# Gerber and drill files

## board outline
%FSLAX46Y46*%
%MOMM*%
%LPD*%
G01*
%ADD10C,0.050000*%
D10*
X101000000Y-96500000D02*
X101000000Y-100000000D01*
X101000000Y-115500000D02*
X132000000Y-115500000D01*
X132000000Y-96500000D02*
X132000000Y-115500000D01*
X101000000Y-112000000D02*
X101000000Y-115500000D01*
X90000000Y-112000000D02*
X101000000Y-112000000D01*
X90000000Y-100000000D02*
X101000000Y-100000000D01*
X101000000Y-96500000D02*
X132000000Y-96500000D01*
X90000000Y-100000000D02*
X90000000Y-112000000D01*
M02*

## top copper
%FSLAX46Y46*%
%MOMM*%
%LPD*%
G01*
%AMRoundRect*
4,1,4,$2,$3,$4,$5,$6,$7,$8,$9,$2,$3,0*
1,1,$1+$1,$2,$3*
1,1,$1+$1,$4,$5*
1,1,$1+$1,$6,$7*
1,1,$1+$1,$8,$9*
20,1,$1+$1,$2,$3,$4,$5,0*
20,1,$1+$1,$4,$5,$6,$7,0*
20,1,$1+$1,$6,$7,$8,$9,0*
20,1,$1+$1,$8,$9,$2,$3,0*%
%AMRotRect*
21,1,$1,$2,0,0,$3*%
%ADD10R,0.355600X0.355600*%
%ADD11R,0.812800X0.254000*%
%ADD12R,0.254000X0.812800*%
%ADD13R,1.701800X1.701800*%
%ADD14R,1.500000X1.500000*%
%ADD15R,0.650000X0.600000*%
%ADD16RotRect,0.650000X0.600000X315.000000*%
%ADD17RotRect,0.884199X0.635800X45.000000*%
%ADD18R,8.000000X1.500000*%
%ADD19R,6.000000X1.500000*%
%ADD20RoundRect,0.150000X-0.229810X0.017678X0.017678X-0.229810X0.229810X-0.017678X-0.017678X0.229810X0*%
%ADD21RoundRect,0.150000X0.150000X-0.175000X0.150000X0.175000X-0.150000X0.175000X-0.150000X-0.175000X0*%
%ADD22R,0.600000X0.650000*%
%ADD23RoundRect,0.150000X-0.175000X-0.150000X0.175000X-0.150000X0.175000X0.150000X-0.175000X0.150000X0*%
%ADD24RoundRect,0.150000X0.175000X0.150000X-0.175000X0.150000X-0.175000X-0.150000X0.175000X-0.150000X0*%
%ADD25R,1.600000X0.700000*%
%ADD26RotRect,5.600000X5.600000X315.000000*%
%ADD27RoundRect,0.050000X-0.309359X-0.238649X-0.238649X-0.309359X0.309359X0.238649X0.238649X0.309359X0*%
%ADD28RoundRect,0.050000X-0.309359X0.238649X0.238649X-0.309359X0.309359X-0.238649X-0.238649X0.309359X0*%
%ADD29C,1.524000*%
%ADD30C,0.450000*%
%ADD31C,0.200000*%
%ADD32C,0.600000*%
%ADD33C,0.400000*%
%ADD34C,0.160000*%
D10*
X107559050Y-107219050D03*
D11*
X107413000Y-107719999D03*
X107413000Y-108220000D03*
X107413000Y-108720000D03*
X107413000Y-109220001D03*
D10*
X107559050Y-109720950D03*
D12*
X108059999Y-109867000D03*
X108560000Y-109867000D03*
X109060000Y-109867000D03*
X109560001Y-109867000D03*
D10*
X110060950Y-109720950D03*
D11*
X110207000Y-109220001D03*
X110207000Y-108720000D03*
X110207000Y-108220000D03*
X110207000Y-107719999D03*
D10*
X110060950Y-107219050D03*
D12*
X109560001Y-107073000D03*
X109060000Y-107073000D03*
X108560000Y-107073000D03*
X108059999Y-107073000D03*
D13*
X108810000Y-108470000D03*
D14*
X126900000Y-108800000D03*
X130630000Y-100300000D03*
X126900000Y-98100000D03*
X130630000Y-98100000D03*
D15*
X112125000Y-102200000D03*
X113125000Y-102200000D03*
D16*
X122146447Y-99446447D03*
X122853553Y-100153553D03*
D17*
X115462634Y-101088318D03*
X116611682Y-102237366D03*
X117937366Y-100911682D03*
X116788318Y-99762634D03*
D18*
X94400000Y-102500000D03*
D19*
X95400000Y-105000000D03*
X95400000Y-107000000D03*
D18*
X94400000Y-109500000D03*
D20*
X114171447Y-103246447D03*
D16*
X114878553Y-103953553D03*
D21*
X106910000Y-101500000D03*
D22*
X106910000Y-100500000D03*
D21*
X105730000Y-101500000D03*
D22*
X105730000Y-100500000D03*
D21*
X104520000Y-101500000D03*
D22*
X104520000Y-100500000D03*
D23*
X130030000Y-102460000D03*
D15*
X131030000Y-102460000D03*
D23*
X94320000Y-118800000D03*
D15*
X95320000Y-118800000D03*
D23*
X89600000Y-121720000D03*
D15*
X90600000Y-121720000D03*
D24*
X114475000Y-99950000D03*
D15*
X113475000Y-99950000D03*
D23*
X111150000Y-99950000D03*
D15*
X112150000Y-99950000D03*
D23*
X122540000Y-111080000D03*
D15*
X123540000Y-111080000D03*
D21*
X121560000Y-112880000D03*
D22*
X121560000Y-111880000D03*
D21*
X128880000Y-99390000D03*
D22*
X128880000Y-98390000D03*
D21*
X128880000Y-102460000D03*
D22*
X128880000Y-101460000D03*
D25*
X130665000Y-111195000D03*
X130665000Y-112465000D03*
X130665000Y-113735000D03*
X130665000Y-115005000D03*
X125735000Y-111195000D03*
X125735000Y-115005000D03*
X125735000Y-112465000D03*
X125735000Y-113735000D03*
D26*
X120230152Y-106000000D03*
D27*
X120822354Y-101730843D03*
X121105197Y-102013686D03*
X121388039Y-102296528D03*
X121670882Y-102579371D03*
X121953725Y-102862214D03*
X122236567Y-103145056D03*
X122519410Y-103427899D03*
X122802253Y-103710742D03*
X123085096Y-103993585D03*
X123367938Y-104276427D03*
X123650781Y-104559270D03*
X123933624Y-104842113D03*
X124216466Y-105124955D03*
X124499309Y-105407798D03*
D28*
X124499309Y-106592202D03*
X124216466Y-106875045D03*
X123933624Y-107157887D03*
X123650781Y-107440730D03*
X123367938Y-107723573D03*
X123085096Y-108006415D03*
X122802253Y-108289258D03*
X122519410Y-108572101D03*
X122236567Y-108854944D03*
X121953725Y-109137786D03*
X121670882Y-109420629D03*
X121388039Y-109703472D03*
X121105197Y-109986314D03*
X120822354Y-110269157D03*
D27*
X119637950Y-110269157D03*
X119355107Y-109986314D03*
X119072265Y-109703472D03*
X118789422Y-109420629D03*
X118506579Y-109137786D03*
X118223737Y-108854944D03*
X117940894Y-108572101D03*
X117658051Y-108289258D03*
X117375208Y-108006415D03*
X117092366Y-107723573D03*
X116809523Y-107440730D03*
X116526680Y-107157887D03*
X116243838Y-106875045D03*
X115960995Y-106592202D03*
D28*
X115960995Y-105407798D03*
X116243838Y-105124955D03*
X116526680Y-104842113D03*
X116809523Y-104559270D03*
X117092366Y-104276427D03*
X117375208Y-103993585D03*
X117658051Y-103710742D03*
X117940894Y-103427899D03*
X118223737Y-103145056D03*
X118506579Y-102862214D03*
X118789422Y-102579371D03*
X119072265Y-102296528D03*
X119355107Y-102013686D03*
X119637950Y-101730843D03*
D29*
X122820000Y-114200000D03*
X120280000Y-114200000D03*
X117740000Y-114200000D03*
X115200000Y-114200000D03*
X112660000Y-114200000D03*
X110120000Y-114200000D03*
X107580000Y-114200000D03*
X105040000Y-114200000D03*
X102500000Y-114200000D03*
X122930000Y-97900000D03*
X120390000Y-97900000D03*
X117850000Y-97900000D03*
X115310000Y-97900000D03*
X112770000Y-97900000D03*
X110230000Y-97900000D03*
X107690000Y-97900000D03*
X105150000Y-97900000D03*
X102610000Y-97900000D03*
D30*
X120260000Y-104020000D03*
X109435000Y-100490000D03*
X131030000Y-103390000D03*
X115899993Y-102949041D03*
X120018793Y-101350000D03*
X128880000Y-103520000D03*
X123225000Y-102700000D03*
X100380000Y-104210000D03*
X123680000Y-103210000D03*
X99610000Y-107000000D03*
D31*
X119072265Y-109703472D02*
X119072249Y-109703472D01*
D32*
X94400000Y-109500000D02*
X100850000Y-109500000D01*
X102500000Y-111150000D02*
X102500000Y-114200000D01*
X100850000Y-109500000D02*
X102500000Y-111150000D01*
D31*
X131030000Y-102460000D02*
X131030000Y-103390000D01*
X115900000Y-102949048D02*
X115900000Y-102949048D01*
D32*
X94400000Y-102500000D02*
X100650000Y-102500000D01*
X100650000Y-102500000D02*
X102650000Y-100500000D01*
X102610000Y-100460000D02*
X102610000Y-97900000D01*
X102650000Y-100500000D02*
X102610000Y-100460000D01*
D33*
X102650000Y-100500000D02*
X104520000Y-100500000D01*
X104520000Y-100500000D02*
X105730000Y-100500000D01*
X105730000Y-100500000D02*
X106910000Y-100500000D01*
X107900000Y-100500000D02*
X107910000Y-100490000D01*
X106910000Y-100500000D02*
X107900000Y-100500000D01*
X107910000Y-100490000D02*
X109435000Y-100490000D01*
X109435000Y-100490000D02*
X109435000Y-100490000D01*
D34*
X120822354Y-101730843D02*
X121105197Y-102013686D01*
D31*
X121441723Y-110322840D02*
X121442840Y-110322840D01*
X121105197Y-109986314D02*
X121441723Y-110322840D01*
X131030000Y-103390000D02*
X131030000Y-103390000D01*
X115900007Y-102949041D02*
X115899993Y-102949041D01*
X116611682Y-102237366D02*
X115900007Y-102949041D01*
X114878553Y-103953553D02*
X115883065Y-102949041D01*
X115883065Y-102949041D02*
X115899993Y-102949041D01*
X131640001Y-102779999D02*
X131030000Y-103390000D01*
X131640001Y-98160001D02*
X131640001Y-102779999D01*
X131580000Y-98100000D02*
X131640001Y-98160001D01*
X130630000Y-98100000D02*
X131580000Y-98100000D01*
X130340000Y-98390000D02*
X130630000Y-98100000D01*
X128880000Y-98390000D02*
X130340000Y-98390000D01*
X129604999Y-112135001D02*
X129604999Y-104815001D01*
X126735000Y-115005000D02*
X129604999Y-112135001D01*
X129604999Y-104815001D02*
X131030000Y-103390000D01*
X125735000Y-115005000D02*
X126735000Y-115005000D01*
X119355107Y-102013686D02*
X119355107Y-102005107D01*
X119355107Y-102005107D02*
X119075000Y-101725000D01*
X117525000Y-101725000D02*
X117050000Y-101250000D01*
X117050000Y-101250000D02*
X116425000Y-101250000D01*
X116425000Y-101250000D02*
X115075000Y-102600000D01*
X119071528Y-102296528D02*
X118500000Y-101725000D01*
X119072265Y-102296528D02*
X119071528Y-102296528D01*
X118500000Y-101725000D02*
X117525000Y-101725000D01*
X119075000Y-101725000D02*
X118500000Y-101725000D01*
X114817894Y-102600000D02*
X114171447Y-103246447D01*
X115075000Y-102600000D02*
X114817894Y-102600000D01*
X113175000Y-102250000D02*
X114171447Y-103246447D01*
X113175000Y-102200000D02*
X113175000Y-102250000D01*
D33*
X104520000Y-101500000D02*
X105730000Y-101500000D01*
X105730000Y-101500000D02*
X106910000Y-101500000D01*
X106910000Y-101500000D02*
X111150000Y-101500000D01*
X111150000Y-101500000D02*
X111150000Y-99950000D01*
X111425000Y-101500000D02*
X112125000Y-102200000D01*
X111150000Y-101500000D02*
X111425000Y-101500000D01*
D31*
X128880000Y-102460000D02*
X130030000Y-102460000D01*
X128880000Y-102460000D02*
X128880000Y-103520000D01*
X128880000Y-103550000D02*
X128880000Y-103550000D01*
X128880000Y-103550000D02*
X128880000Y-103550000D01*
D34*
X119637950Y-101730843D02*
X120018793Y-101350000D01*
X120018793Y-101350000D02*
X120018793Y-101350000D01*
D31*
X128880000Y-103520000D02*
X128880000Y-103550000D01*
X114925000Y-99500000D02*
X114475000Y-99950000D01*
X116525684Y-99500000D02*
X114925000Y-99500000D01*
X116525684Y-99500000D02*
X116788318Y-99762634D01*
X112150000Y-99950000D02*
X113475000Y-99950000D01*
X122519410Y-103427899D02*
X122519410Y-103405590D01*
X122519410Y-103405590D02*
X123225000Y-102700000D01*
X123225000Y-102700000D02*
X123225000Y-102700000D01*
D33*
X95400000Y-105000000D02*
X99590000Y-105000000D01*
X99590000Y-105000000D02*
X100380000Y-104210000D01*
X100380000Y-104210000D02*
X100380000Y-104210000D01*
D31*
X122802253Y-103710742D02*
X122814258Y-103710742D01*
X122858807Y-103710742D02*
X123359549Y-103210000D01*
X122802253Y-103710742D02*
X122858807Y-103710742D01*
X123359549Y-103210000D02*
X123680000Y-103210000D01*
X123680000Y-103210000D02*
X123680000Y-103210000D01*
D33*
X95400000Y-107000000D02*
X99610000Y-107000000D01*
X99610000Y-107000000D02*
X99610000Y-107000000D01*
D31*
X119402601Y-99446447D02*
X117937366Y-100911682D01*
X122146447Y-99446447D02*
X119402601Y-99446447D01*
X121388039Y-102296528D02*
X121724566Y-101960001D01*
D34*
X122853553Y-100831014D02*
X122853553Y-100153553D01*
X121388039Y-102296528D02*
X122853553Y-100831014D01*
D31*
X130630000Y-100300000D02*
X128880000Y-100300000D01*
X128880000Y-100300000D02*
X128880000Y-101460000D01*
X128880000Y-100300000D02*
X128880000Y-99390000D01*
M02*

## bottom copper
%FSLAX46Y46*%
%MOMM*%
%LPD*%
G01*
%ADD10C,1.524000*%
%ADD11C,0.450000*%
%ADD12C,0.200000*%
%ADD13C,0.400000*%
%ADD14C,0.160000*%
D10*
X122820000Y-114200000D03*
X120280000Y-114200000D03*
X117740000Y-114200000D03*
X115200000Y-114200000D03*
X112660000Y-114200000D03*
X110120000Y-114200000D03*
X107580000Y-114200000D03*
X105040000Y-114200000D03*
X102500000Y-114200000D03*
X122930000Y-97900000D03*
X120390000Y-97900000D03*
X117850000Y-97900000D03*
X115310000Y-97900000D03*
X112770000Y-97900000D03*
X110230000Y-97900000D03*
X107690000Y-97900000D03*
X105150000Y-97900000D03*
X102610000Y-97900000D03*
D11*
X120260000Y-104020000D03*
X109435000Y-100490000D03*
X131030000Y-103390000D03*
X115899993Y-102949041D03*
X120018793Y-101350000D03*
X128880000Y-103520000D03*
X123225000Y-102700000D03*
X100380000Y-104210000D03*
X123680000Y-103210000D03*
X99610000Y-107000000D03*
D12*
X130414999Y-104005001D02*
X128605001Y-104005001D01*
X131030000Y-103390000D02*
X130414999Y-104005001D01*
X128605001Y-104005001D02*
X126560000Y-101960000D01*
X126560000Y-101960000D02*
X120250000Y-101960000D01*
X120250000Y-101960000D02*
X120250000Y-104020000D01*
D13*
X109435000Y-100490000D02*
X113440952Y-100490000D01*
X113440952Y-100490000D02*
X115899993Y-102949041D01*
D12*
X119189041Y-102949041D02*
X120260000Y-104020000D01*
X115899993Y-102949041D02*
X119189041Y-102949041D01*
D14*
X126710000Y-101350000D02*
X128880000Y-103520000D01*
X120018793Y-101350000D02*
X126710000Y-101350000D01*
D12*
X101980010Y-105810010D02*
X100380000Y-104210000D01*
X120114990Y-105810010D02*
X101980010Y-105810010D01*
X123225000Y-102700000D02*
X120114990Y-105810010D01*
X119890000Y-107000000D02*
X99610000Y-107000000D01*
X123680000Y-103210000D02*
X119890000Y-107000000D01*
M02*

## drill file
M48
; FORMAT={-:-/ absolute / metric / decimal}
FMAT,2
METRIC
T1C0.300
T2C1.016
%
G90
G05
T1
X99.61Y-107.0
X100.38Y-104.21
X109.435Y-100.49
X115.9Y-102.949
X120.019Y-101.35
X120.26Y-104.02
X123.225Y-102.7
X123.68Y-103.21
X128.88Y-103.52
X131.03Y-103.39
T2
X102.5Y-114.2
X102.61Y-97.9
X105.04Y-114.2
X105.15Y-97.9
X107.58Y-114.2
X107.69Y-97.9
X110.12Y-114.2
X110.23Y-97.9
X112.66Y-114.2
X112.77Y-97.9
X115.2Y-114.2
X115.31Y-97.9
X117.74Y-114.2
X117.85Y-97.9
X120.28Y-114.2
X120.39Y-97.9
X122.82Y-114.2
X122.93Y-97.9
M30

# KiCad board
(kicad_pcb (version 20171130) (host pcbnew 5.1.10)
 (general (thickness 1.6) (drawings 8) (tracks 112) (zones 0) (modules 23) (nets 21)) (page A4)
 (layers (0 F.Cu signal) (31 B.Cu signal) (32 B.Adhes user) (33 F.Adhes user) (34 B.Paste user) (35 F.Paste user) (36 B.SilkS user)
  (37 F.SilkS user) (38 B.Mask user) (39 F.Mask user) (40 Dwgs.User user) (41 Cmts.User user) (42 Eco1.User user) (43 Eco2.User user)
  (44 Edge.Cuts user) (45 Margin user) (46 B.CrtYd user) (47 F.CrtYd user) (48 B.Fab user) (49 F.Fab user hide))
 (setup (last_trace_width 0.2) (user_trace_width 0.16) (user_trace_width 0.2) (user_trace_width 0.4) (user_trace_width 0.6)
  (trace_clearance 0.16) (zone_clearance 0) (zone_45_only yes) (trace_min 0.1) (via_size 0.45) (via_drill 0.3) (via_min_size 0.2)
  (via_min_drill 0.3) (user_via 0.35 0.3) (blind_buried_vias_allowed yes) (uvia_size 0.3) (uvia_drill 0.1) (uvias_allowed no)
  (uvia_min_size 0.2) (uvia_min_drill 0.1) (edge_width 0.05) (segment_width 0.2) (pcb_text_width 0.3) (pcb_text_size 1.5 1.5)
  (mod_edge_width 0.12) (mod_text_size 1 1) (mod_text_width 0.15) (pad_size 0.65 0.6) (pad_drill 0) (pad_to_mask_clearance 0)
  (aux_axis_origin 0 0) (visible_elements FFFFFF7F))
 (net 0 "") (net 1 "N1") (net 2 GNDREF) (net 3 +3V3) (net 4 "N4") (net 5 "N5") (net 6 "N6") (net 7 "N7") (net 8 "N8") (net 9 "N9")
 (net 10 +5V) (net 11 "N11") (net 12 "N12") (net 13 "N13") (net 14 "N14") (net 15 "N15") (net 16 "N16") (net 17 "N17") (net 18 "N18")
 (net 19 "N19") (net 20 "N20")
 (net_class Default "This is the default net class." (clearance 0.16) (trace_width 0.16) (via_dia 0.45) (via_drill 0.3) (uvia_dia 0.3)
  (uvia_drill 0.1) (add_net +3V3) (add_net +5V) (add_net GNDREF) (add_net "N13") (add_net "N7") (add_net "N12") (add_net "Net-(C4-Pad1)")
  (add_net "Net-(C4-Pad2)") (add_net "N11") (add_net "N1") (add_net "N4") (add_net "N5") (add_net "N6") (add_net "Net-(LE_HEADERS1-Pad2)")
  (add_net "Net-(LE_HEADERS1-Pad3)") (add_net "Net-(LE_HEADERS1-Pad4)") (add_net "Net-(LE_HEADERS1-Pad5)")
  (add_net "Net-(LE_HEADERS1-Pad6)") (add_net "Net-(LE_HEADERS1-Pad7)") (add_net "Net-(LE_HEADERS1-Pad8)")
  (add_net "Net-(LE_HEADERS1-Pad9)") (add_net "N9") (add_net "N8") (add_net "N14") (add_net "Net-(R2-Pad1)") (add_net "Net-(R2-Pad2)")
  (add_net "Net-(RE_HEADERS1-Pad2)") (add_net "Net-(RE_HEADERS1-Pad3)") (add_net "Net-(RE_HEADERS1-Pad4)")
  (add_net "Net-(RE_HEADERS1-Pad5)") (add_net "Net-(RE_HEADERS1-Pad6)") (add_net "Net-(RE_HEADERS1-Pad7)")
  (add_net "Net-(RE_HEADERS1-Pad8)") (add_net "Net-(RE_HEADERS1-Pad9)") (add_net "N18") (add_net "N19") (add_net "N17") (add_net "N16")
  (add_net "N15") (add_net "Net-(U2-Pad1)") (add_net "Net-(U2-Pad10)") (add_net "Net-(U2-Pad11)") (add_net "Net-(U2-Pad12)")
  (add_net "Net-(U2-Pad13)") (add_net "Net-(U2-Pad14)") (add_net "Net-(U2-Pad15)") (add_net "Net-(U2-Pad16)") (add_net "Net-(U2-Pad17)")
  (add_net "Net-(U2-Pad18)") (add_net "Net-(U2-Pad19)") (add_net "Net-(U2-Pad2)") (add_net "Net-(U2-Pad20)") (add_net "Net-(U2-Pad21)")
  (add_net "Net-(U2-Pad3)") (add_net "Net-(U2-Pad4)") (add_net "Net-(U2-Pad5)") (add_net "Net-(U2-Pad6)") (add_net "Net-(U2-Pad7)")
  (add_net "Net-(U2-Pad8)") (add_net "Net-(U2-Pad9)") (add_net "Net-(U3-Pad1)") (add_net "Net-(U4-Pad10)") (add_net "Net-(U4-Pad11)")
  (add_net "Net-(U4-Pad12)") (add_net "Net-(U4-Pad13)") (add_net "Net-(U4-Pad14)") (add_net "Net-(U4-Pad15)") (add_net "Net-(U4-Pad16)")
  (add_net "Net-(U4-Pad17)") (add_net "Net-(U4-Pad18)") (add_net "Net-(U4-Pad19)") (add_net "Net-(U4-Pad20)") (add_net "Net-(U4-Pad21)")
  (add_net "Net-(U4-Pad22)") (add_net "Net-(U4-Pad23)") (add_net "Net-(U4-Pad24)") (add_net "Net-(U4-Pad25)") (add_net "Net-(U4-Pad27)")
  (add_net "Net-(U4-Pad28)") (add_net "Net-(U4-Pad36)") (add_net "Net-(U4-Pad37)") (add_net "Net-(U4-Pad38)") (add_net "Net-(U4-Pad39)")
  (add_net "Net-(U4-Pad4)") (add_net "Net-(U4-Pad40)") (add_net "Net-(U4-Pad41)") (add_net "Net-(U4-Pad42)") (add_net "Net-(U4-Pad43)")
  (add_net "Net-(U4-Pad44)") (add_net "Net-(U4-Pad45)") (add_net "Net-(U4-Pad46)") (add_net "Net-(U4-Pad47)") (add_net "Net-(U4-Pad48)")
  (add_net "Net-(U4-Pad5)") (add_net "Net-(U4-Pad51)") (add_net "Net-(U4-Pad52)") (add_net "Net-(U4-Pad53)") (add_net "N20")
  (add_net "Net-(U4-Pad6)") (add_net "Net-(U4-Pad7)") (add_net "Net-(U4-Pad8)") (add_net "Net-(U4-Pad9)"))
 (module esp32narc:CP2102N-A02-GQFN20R (layer F.Cu) (at 108.81 108.47)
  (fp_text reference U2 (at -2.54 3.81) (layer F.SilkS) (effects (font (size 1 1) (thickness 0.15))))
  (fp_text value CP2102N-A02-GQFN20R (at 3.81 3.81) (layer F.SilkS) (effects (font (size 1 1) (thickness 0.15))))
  (pad 1 smd rect (at -1.25095 -1.25095) (size 0.3556 0.3556) (layers F.Cu F.Paste F.Mask))
  (pad 2 smd rect (at -1.397 -0.750001 90) (size 0.254 0.8128) (layers F.Cu F.Paste F.Mask))
  (pad 3 smd rect (at -1.397 -0.25 90) (size 0.254 0.8128) (layers F.Cu F.Paste F.Mask))
  (pad 4 smd rect (at -1.397 0.25 90) (size 0.254 0.8128) (layers F.Cu F.Paste F.Mask))
  (pad 5 smd rect (at -1.397 0.750001 90) (size 0.254 0.8128) (layers F.Cu F.Paste F.Mask))
  (pad 6 smd rect (at -1.25095 1.25095) (size 0.3556 0.3556) (layers F.Cu F.Paste F.Mask))
  (pad 7 smd rect (at -0.750001 1.397) (size 0.254 0.8128) (layers F.Cu F.Paste F.Mask))
  (pad 8 smd rect (at -0.25 1.397) (size 0.254 0.8128) (layers F.Cu F.Paste F.Mask))
  (pad 9 smd rect (at 0.25 1.397) (size 0.254 0.8128) (layers F.Cu F.Paste F.Mask))
  (pad 10 smd rect (at 0.750001 1.397) (size 0.254 0.8128) (layers F.Cu F.Paste F.Mask))
  (pad 11 smd rect (at 1.25095 1.25095) (size 0.3556 0.3556) (layers F.Cu F.Paste F.Mask))
  (pad 12 smd rect (at 1.397 0.750001 90) (size 0.254 0.8128) (layers F.Cu F.Paste F.Mask))
  (pad 13 smd rect (at 1.397 0.25 90) (size 0.254 0.8128) (layers F.Cu F.Paste F.Mask))
  (pad 14 smd rect (at 1.397 -0.25 90) (size 0.254 0.8128) (layers F.Cu F.Paste F.Mask))
  (pad 15 smd rect (at 1.397 -0.750001 90) (size 0.254 0.8128) (layers F.Cu F.Paste F.Mask))
  (pad 16 smd rect (at 1.25095 -1.25095) (size 0.3556 0.3556) (layers F.Cu F.Paste F.Mask))
  (pad 17 smd rect (at 0.750001 -1.397) (size 0.254 0.8128) (layers F.Cu F.Paste F.Mask))
  (pad 18 smd rect (at 0.25 -1.397) (size 0.254 0.8128) (layers F.Cu F.Paste F.Mask))
  (pad 19 smd rect (at -0.25 -1.397) (size 0.254 0.8128) (layers F.Cu F.Paste F.Mask))
  (pad 20 smd rect (at -0.750001 -1.397) (size 0.254 0.8128) (layers F.Cu F.Paste F.Mask))
  (pad 21 smd rect (at 0 0) (size 1.7018 1.7018) (layers F.Cu F.Paste F.Mask)))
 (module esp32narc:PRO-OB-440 (layer F.Cu) (at 130.63 98.1 270)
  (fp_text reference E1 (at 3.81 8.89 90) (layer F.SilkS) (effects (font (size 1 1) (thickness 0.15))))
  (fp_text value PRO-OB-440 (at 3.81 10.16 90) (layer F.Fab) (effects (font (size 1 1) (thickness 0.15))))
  (pad 4 smd rect (at 10.7 3.73 270) (size 1.5 1.5) (layers F.Cu F.Paste F.Mask) (clearance 0.75))
  (pad 2 smd rect (at 2.2 0 270) (size 1.5 1.5) (layers F.Cu F.Paste F.Mask) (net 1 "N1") (clearance 0.15))
  (pad 3 smd rect (at 0 3.73 270) (size 1.5 1.5) (layers F.Cu F.Paste F.Mask) (clearance 0.55))
  (pad 1 smd rect (at 0 0 270) (size 1.5 1.5) (layers F.Cu F.Paste F.Mask) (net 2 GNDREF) (clearance 0.15)))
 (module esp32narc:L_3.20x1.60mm (layer F.Cu) (at 112.625 102.2)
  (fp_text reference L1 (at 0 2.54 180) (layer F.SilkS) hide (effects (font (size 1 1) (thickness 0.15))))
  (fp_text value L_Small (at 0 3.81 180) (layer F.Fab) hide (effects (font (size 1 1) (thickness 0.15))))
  (pad 1 smd rect (at -0.5 0) (size 0.65 0.6) (layers F.Cu F.Paste F.Mask) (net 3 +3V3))
  (pad 2 smd rect (at 0.5 0) (size 0.65 0.6) (layers F.Cu F.Paste F.Mask) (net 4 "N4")))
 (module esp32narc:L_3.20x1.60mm (layer F.Cu) (at 122.5 99.8 315)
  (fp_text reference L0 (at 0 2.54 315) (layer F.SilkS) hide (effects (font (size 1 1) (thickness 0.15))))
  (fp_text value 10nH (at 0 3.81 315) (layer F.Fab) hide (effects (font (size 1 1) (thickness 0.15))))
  (pad 1 smd rect (at -0.5 0 315) (size 0.65 0.6) (layers F.Cu F.Paste F.Mask) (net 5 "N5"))
  (pad 2 smd rect (at 0.5 0 315) (size 0.65 0.6) (layers F.Cu F.Paste F.Mask) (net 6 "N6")))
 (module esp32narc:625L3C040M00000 (layer F.Cu) (at 116.7 101 45)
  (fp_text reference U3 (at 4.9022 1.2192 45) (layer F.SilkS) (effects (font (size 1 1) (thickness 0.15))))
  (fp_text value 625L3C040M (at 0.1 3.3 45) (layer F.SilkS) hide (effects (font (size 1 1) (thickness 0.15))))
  (pad 1 smd rect (at -0.9374 -0.8125 45) (size 0.884199 0.6358) (layers F.Cu F.Paste F.Mask))
  (pad 2 smd rect (at -0.9374 0.8125 45) (size 0.884199 0.6358) (layers F.Cu F.Paste F.Mask) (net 2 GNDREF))
  (pad 3 smd rect (at 0.9374 0.8125 45) (size 0.884199 0.6358) (layers F.Cu F.Paste F.Mask) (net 5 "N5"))
  (pad 4 smd rect (at 0.9374 -0.8125 45) (size 0.884199 0.6358) (layers F.Cu F.Paste F.Mask) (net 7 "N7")))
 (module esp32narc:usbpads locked (layer F.Cu) (at 98.4 106 90)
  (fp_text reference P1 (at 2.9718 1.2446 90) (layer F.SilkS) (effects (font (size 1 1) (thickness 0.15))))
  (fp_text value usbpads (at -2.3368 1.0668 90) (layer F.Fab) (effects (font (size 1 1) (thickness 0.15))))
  (pad P4 smd rect (at 3.5 -4 90) (size 1.5 8) (layers F.Cu F.Paste F.Mask) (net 2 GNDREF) (solder_mask_margin 0.105) (clearance 0.55))
  (pad P3 smd rect (at 1 -3 90) (size 1.5 6) (layers F.Cu F.Paste F.Mask) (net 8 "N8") (clearance 0.55))
  (pad P2 smd rect (at -1 -3 90) (size 1.5 6) (layers F.Cu F.Paste F.Mask) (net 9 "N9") (clearance 0.55))
  (pad P1 smd rect (at -3.5 -4 90) (size 1.5 8) (layers F.Cu F.Paste F.Mask) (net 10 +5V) (solder_mask_margin 0.105) (clearance 0.55)))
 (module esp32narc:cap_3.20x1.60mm (layer F.Cu) (at 114.525 103.6 315)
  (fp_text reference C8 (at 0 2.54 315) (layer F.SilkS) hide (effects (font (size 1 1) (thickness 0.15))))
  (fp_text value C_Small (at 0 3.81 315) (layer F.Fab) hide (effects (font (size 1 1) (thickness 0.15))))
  (pad 1 smd roundrect (at -0.5 0 315) (size 0.65 0.6) (layers F.Cu F.Paste F.Mask) (roundrect_rratio 0.25) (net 4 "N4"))
  (pad 2 smd rect (at 0.5 0 315) (size 0.65 0.6) (layers F.Cu F.Paste F.Mask) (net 2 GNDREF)))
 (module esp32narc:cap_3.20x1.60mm (layer F.Cu) (at 106.91 101 90)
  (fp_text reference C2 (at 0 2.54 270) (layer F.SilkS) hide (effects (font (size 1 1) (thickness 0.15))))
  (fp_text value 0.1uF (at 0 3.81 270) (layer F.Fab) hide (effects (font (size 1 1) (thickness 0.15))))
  (pad 1 smd roundrect (at -0.5 0 90) (size 0.65 0.6) (layers F.Cu F.Paste F.Mask) (roundrect_rratio 0.25) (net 3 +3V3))
  (pad 2 smd rect (at 0.5 0 90) (size 0.65 0.6) (layers F.Cu F.Paste F.Mask) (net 2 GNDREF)))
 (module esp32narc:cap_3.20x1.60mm (layer F.Cu) (at 105.73 101 90)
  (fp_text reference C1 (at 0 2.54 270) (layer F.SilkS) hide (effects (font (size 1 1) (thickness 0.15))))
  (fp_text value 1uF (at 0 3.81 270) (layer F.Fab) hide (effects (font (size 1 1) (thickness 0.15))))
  (pad 1 smd roundrect (at -0.5 0 90) (size 0.65 0.6) (layers F.Cu F.Paste F.Mask) (roundrect_rratio 0.25) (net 3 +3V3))
  (pad 2 smd rect (at 0.5 0 90) (size 0.65 0.6) (layers F.Cu F.Paste F.Mask) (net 2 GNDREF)))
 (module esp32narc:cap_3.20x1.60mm (layer F.Cu) (at 104.52 101 90)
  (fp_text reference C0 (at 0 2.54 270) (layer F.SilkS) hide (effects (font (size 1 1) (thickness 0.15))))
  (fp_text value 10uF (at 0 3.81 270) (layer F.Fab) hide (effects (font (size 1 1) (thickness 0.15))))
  (pad 1 smd roundrect (at -0.5 0 90) (size 0.65 0.6) (layers F.Cu F.Paste F.Mask) (roundrect_rratio 0.25) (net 3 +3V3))
  (pad 2 smd rect (at 0.5 0 90) (size 0.65 0.6) (layers F.Cu F.Paste F.Mask) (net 2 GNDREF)))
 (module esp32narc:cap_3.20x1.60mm (layer F.Cu) (at 130.53 102.46)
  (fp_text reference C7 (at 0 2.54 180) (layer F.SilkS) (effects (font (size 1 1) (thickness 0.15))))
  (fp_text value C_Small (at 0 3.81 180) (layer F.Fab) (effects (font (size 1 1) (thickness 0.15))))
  (pad 1 smd roundrect (at -0.5 0) (size 0.65 0.6) (layers F.Cu F.Paste F.Mask) (roundrect_rratio 0.25) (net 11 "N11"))
  (pad 2 smd rect (at 0.5 0) (size 0.65 0.6) (layers F.Cu F.Paste F.Mask) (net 2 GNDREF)))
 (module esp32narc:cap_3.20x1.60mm (layer F.Cu) (at 94.82 118.8)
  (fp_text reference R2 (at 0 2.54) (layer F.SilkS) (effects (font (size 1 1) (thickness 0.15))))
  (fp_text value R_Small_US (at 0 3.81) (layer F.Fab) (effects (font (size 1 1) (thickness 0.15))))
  (pad 1 smd roundrect (at -0.5 0) (size 0.65 0.6) (layers F.Cu F.Paste F.Mask) (roundrect_rratio 0.25))
  (pad 2 smd rect (at 0.5 0) (size 0.65 0.6) (layers F.Cu F.Paste F.Mask)))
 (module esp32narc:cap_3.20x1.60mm (layer F.Cu) (at 90.1 121.72)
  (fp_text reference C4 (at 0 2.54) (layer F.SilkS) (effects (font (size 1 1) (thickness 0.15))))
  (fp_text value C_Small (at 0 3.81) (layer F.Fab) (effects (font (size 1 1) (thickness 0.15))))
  (pad 1 smd roundrect (at -0.5 0) (size 0.65 0.6) (layers F.Cu F.Paste F.Mask) (roundrect_rratio 0.25))
  (pad 2 smd rect (at 0.5 0) (size 0.65 0.6) (layers F.Cu F.Paste F.Mask)))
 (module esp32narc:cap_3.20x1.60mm (layer F.Cu) (at 113.975 99.95 180)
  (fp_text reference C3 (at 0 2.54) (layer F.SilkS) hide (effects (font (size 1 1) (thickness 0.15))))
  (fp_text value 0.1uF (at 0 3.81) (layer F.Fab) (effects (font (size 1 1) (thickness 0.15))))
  (pad 1 smd roundrect (at -0.5 0 180) (size 0.65 0.6) (layers F.Cu F.Paste F.Mask) (roundrect_rratio 0.25) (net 7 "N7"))
  (pad 2 smd rect (at 0.5 0 180) (size 0.65 0.6) (layers F.Cu F.Paste F.Mask) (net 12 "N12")))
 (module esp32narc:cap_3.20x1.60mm (layer F.Cu) (at 111.65 99.95)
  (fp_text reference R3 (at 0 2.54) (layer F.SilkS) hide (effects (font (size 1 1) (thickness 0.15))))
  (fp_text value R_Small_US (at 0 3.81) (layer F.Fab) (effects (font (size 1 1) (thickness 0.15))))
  (pad 1 smd roundrect (at -0.5 0) (size 0.65 0.6) (layers F.Cu F.Paste F.Mask) (roundrect_rratio 0.25) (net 3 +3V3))
  (pad 2 smd rect (at 0.5 0) (size 0.65 0.6) (layers F.Cu F.Paste F.Mask) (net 12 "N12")))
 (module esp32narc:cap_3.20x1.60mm (layer F.Cu) (at 123.04 111.08)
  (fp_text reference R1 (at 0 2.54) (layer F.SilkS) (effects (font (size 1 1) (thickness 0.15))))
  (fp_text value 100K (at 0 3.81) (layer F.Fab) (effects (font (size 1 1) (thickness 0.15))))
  (pad 1 smd roundrect (at -0.5 0) (size 0.65 0.6) (layers F.Cu F.Paste F.Mask) (roundrect_rratio 0.25) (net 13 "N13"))
  (pad 2 smd rect (at 0.5 0) (size 0.65 0.6) (layers F.Cu F.Paste F.Mask) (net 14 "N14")))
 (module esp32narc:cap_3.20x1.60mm (layer F.Cu) (at 121.56 112.38 90)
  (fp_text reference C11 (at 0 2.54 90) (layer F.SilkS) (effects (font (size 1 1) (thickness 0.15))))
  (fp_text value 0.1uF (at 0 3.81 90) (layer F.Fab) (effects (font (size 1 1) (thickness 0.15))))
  (pad 1 smd roundrect (at -0.5 0 90) (size 0.65 0.6) (layers F.Cu F.Paste F.Mask) (roundrect_rratio 0.25) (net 2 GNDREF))
  (pad 2 smd rect (at 0.5 0 90) (size 0.65 0.6) (layers F.Cu F.Paste F.Mask) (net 13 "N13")))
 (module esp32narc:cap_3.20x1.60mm (layer F.Cu) (at 128.88 98.89 90)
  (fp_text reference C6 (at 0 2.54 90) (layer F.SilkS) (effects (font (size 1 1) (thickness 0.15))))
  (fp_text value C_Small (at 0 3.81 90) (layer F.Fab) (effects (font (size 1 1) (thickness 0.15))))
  (pad 1 smd roundrect (at -0.5 0 90) (size 0.65 0.6) (layers F.Cu F.Paste F.Mask) (roundrect_rratio 0.25) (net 1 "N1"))
  (pad 2 smd rect (at 0.5 0 90) (size 0.65 0.6) (layers F.Cu F.Paste F.Mask) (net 2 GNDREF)))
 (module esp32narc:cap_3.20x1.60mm (layer F.Cu) (at 128.88 101.96 90)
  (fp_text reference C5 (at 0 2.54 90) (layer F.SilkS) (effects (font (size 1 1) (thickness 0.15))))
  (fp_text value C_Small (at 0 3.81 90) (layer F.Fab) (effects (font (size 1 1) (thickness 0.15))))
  (pad 1 smd roundrect (at -0.5 0 90) (size 0.65 0.6) (layers F.Cu F.Paste F.Mask) (roundrect_rratio 0.25) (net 11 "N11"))
  (pad 2 smd rect (at 0.5 0 90) (size 0.65 0.6) (layers F.Cu F.Paste F.Mask) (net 1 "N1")))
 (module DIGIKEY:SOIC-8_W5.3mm (layer F.Cu) (at 128.2 113.1)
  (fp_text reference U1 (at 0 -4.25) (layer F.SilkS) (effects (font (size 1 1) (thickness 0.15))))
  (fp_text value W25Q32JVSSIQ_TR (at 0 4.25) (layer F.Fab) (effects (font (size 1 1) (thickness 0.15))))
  (pad 8 smd rect (at 2.465 -1.905) (size 1.6 0.7) (layers F.Cu F.Paste F.Mask) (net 13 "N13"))
  (pad 7 smd rect (at 2.465 -0.635) (size 1.6 0.7) (layers F.Cu F.Paste F.Mask) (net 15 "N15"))
  (pad 6 smd rect (at 2.465 0.635) (size 1.6 0.7) (layers F.Cu F.Paste F.Mask) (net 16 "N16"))
  (pad 5 smd rect (at 2.465 1.905) (size 1.6 0.7) (layers F.Cu F.Paste F.Mask) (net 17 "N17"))
  (pad 1 smd rect (at -2.465 -1.905) (size 1.6 0.7) (layers F.Cu F.Paste F.Mask) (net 14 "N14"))
  (pad 4 smd rect (at -2.465 1.905) (size 1.6 0.7) (layers F.Cu F.Paste F.Mask) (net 2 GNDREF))
  (pad 2 smd rect (at -2.465 -0.635) (size 1.6 0.7) (layers F.Cu F.Paste F.Mask) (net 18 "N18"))
  (pad 3 smd rect (at -2.465 0.635) (size 1.6 0.7) (layers F.Cu F.Paste F.Mask) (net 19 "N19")))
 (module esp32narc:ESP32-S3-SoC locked (layer F.Cu) (at 120.230152 106 315)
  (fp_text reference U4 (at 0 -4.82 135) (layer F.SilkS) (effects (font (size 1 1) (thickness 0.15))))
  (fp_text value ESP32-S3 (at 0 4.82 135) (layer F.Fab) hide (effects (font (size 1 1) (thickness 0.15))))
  (pad "" smd roundrect (at 2.1 2.1 315) (size 1.13 1.13) (layers F.Paste) (roundrect_rratio 0.221239))
  (pad "" smd roundrect (at 2.1 0.7 315) (size 1.13 1.13) (layers F.Paste) (roundrect_rratio 0.221239))
  (pad "" smd roundrect (at 2.1 -0.7 315) (size 1.13 1.13) (layers F.Paste) (roundrect_rratio 0.221239))
  (pad "" smd roundrect (at 2.1 -2.1 315) (size 1.13 1.13) (layers F.Paste) (roundrect_rratio 0.221239))
  (pad "" smd roundrect (at 0.7 2.1 315) (size 1.13 1.13) (layers F.Paste) (roundrect_rratio 0.221239))
  (pad "" smd roundrect (at 0.7 0.7 315) (size 1.13 1.13) (layers F.Paste) (roundrect_rratio 0.221239))
  (pad "" smd roundrect (at 0.7 -0.7 315) (size 1.13 1.13) (layers F.Paste) (roundrect_rratio 0.221239))
  (pad "" smd roundrect (at 0.7 -2.1 315) (size 1.13 1.13) (layers F.Paste) (roundrect_rratio 0.221239))
  (pad "" smd roundrect (at -0.7 2.1 315) (size 1.13 1.13) (layers F.Paste) (roundrect_rratio 0.221239))
  (pad "" smd roundrect (at -0.7 0.7 315) (size 1.13 1.13) (layers F.Paste) (roundrect_rratio 0.221239))
  (pad "" smd roundrect (at -0.7 -0.7 315) (size 1.13 1.13) (layers F.Paste) (roundrect_rratio 0.221239))
  (pad "" smd roundrect (at -0.7 -2.1 315) (size 1.13 1.13) (layers F.Paste) (roundrect_rratio 0.221239))
  (pad "" smd roundrect (at -2.1 2.1 315) (size 1.13 1.13) (layers F.Paste) (roundrect_rratio 0.221239))
  (pad "" smd roundrect (at -2.1 0.7 315) (size 1.13 1.13) (layers F.Paste) (roundrect_rratio 0.221239))
  (pad "" smd roundrect (at -2.1 -0.7 315) (size 1.13 1.13) (layers F.Paste) (roundrect_rratio 0.221239))
  (pad "" smd roundrect (at -2.1 -2.1 315) (size 1.13 1.13) (layers F.Paste) (roundrect_rratio 0.221239))
  (pad 57 smd rect (at 0 0 315) (size 5.6 5.6) (layers F.Cu F.Mask) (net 2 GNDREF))
  (pad 56 smd roundrect (at -2.6 -3.4375 315) (size 0.2 0.875) (layers F.Cu F.Paste F.Mask) (roundrect_rratio 0.25) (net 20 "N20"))
  (pad 55 smd roundrect (at -2.2 -3.4375 315) (size 0.2 0.875) (layers F.Cu F.Paste F.Mask) (roundrect_rratio 0.25) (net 20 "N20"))
  (pad 54 smd roundrect (at -1.8 -3.4375 315) (size 0.2 0.875) (layers F.Cu F.Paste F.Mask) (roundrect_rratio 0.25) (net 6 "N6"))
  (pad 53 smd roundrect (at -1.4 -3.4375 315) (size 0.2 0.875) (layers F.Cu F.Paste F.Mask) (roundrect_rratio 0.25))
  (pad 52 smd roundrect (at -1 -3.4375 315) (size 0.2 0.875) (layers F.Cu F.Paste F.Mask) (roundrect_rratio 0.25))
  (pad 51 smd roundrect (at -0.6 -3.4375 315) (size 0.2 0.875) (layers F.Cu F.Paste F.Mask) (roundrect_rratio 0.25))
  (pad 50 smd roundrect (at -0.2 -3.4375 315) (size 0.2 0.875) (layers F.Cu F.Paste F.Mask) (roundrect_rratio 0.25) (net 8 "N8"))
  (pad 49 smd roundrect (at 0.2 -3.4375 315) (size 0.2 0.875) (layers F.Cu F.Paste F.Mask) (roundrect_rratio 0.25) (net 9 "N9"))
  (pad 48 smd roundrect (at 0.6 -3.4375 315) (size 0.2 0.875) (layers F.Cu F.Paste F.Mask) (roundrect_rratio 0.25))
  (pad 47 smd roundrect (at 1 -3.4375 315) (size 0.2 0.875) (layers F.Cu F.Paste F.Mask) (roundrect_rratio 0.25))
  (pad 46 smd roundrect (at 1.4 -3.4375 315) (size 0.2 0.875) (layers F.Cu F.Paste F.Mask) (roundrect_rratio 0.25))
  (pad 45 smd roundrect (at 1.8 -3.4375 315) (size 0.2 0.875) (layers F.Cu F.Paste F.Mask) (roundrect_rratio 0.25))
  (pad 44 smd roundrect (at 2.2 -3.4375 315) (size 0.2 0.875) (layers F.Cu F.Paste F.Mask) (roundrect_rratio 0.25))
  (pad 43 smd roundrect (at 2.6 -3.4375 315) (size 0.2 0.875) (layers F.Cu F.Paste F.Mask) (roundrect_rratio 0.25))
  (pad 42 smd roundrect (at 3.4375 -2.6 315) (size 0.875 0.2) (layers F.Cu F.Paste F.Mask) (roundrect_rratio 0.25))
  (pad 41 smd roundrect (at 3.4375 -2.2 315) (size 0.875 0.2) (layers F.Cu F.Paste F.Mask) (roundrect_rratio 0.25))
  (pad 40 smd roundrect (at 3.4375 -1.8 315) (size 0.875 0.2) (layers F.Cu F.Paste F.Mask) (roundrect_rratio 0.25))
  (pad 39 smd roundrect (at 3.4375 -1.4 315) (size 0.875 0.2) (layers F.Cu F.Paste F.Mask) (roundrect_rratio 0.25))
  (pad 38 smd roundrect (at 3.4375 -1 315) (size 0.875 0.2) (layers F.Cu F.Paste F.Mask) (roundrect_rratio 0.25))
  (pad 37 smd roundrect (at 3.4375 -0.6 315) (size 0.875 0.2) (layers F.Cu F.Paste F.Mask) (roundrect_rratio 0.25))
  (pad 36 smd roundrect (at 3.4375 -0.2 315) (size 0.875 0.2) (layers F.Cu F.Paste F.Mask) (roundrect_rratio 0.25))
  (pad 35 smd roundrect (at 3.4375 0.2 315) (size 0.875 0.2) (layers F.Cu F.Paste F.Mask) (roundrect_rratio 0.25) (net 17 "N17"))
  (pad 34 smd roundrect (at 3.4375 0.6 315) (size 0.875 0.2) (layers F.Cu F.Paste F.Mask) (roundrect_rratio 0.25) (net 18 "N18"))
  (pad 33 smd roundrect (at 3.4375 1 315) (size 0.875 0.2) (layers F.Cu F.Paste F.Mask) (roundrect_rratio 0.25) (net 16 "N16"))
  (pad 32 smd roundrect (at 3.4375 1.4 315) (size 0.875 0.2) (layers F.Cu F.Paste F.Mask) (roundrect_rratio 0.25) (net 14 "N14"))
  (pad 31 smd roundrect (at 3.4375 1.8 315) (size 0.875 0.2) (layers F.Cu F.Paste F.Mask) (roundrect_rratio 0.25) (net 19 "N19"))
  (pad 30 smd roundrect (at 3.4375 2.2 315) (size 0.875 0.2) (layers F.Cu F.Paste F.Mask) (roundrect_rratio 0.25) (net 15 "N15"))
  (pad 29 smd roundrect (at 3.4375 2.6 315) (size 0.875 0.2) (layers F.Cu F.Paste F.Mask) (roundrect_rratio 0.25) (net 13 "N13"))
  (pad 28 smd roundrect (at 2.6 3.4375 315) (size 0.2 0.875) (layers F.Cu F.Paste F.Mask) (roundrect_rratio 0.25))
  (pad 27 smd roundrect (at 2.2 3.4375 315) (size 0.2 0.875) (layers F.Cu F.Paste F.Mask) (roundrect_rratio 0.25))
  (pad 26 smd roundrect (at 1.8 3.4375 315) (size 0.2 0.875) (layers F.Cu F.Paste F.Mask) (roundrect_rratio 0.25))
  (pad 25 smd roundrect (at 1.4 3.4375 315) (size 0.2 0.875) (layers F.Cu F.Paste F.Mask) (roundrect_rratio 0.25))
  (pad 24 smd roundrect (at 1 3.4375 315) (size 0.2 0.875) (layers F.Cu F.Paste F.Mask) (roundrect_rratio 0.25))
  (pad 23 smd roundrect (at 0.6 3.4375 315) (size 0.2 0.875) (layers F.Cu F.Paste F.Mask) (roundrect_rratio 0.25))
  (pad 22 smd roundrect (at 0.2 3.4375 315) (size 0.2 0.875) (layers F.Cu F.Paste F.Mask) (roundrect_rratio 0.25))
  (pad 21 smd roundrect (at -0.2 3.4375 315) (size 0.2 0.875) (layers F.Cu F.Paste F.Mask) (roundrect_rratio 0.25))
  (pad 20 smd roundrect (at -0.6 3.4375 315) (size 0.2 0.875) (layers F.Cu F.Paste F.Mask) (roundrect_rratio 0.25))
  (pad 19 smd roundrect (at -1 3.4375 315) (size 0.2 0.875) (layers F.Cu F.Paste F.Mask) (roundrect_rratio 0.25))
  (pad 18 smd roundrect (at -1.4 3.4375 315) (size 0.2 0.875) (layers F.Cu F.Paste F.Mask) (roundrect_rratio 0.25))
  (pad 17 smd roundrect (at -1.8 3.4375 315) (size 0.2 0.875) (layers F.Cu F.Paste F.Mask) (roundrect_rratio 0.25))
  (pad 16 smd roundrect (at -2.2 3.4375 315) (size 0.2 0.875) (layers F.Cu F.Paste F.Mask) (roundrect_rratio 0.25))
  (pad 15 smd roundrect (at -2.6 3.4375 315) (size 0.2 0.875) (layers F.Cu F.Paste F.Mask) (roundrect_rratio 0.25))
  (pad 14 smd roundrect (at -3.4375 2.6 315) (size 0.875 0.2) (layers F.Cu F.Paste F.Mask) (roundrect_rratio 0.25))
  (pad 13 smd roundrect (at -3.4375 2.2 315) (size 0.875 0.2) (layers F.Cu F.Paste F.Mask) (roundrect_rratio 0.25))
  (pad 12 smd roundrect (at -3.4375 1.8 315) (size 0.875 0.2) (layers F.Cu F.Paste F.Mask) (roundrect_rratio 0.25))
  (pad 11 smd roundrect (at -3.4375 1.4 315) (size 0.875 0.2) (layers F.Cu F.Paste F.Mask) (roundrect_rratio 0.25))
  (pad 10 smd roundrect (at -3.4375 1 315) (size 0.875 0.2) (layers F.Cu F.Paste F.Mask) (roundrect_rratio 0.25))
  (pad 9 smd roundrect (at -3.4375 0.6 315) (size 0.875 0.2) (layers F.Cu F.Paste F.Mask) (roundrect_rratio 0.25))
  (pad 8 smd roundrect (at -3.4375 0.2 315) (size 0.875 0.2) (layers F.Cu F.Paste F.Mask) (roundrect_rratio 0.25))
  (pad 7 smd roundrect (at -3.4375 -0.2 315) (size 0.875 0.2) (layers F.Cu F.Paste F.Mask) (roundrect_rratio 0.25))
  (pad 6 smd roundrect (at -3.4375 -0.6 315) (size 0.875 0.2) (layers F.Cu F.Paste F.Mask) (roundrect_rratio 0.25))
  (pad 5 smd roundrect (at -3.4375 -1 315) (size 0.875 0.2) (layers F.Cu F.Paste F.Mask) (roundrect_rratio 0.25))
  (pad 4 smd roundrect (at -3.4375 -1.4 315) (size 0.875 0.2) (layers F.Cu F.Paste F.Mask) (roundrect_rratio 0.25))
  (pad 3 smd roundrect (at -3.4375 -1.8 315) (size 0.875 0.2) (layers F.Cu F.Paste F.Mask) (roundrect_rratio 0.25) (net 4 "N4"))
  (pad 2 smd roundrect (at -3.4375 -2.2 315) (size 0.875 0.2) (layers F.Cu F.Paste F.Mask) (roundrect_rratio 0.25) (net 4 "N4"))
  (pad 1 smd roundrect (at -3.4375 -2.6 315) (size 0.875 0.2) (layers F.Cu F.Paste F.Mask) (roundrect_rratio 0.25) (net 11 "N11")))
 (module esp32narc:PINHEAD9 (layer F.Cu) (at 111.39 114.2)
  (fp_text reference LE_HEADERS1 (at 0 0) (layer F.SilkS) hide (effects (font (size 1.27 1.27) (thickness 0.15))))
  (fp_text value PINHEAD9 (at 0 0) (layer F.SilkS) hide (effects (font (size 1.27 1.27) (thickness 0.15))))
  (pad 9 thru_hole circle (at 11.43 0) (size 1.524 1.524) (drill 1.016) (layers *.Cu *.Mask) (solder_mask_margin 0.1016))
  (pad 8 thru_hole circle (at 8.89 0) (size 1.524 1.524) (drill 1.016) (layers *.Cu *.Mask) (solder_mask_margin 0.1016))
  (pad 7 thru_hole circle (at 6.35 0) (size 1.524 1.524) (drill 1.016) (layers *.Cu *.Mask) (solder_mask_margin 0.1016))
  (pad 6 thru_hole circle (at 3.81 0) (size 1.524 1.524) (drill 1.016) (layers *.Cu *.Mask) (solder_mask_margin 0.1016))
  (pad 5 thru_hole circle (at 1.27 0) (size 1.524 1.524) (drill 1.016) (layers *.Cu *.Mask) (solder_mask_margin 0.1016))
  (pad 4 thru_hole circle (at -1.27 0) (size 1.524 1.524) (drill 1.016) (layers *.Cu *.Mask) (solder_mask_margin 0.1016))
  (pad 3 thru_hole circle (at -3.81 0) (size 1.524 1.524) (drill 1.016) (layers *.Cu *.Mask) (solder_mask_margin 0.1016))
  (pad 2 thru_hole circle (at -6.35 0) (size 1.524 1.524) (drill 1.016) (layers *.Cu *.Mask) (solder_mask_margin 0.1016))
  (pad 1 thru_hole circle (at -8.89 0) (size 1.524 1.524) (drill 1.016) (layers *.Cu *.Mask) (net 10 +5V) (solder_mask_margin 0.1016)))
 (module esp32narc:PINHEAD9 (layer F.Cu) (at 111.5 97.9)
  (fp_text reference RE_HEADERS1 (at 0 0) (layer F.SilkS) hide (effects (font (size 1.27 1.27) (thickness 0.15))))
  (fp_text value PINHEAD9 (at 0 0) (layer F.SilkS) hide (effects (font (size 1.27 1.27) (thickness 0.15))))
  (pad 9 thru_hole circle (at 11.43 0) (size 1.524 1.524) (drill 1.016) (layers *.Cu *.Mask) (solder_mask_margin 0.1016))
  (pad 8 thru_hole circle (at 8.89 0) (size 1.524 1.524) (drill 1.016) (layers *.Cu *.Mask) (solder_mask_margin 0.1016))
  (pad 7 thru_hole circle (at 6.35 0) (size 1.524 1.524) (drill 1.016) (layers *.Cu *.Mask) (solder_mask_margin 0.1016))
  (pad 6 thru_hole circle (at 3.81 0) (size 1.524 1.524) (drill 1.016) (layers *.Cu *.Mask) (solder_mask_margin 0.1016))
  (pad 5 thru_hole circle (at 1.27 0) (size 1.524 1.524) (drill 1.016) (layers *.Cu *.Mask) (solder_mask_margin 0.1016))
  (pad 4 thru_hole circle (at -1.27 0) (size 1.524 1.524) (drill 1.016) (layers *.Cu *.Mask) (solder_mask_margin 0.1016))
  (pad 3 thru_hole circle (at -3.81 0) (size 1.524 1.524) (drill 1.016) (layers *.Cu *.Mask) (solder_mask_margin 0.1016))
  (pad 2 thru_hole circle (at -6.35 0) (size 1.524 1.524) (drill 1.016) (layers *.Cu *.Mask) (solder_mask_margin 0.1016))
  (pad 1 thru_hole circle (at -8.89 0) (size 1.524 1.524) (drill 1.016) (layers *.Cu *.Mask) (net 2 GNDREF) (solder_mask_margin 0.1016)))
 (gr_line (start 101 96.5) (end 101 100) (layer Edge.Cuts) (width 0.05))
 (gr_line (start 101 115.5) (end 132 115.5) (layer Edge.Cuts) (width 0.05))
 (gr_line (start 132 96.5) (end 132 115.5) (layer Edge.Cuts) (width 0.05))
 (gr_line (start 101 112) (end 101 115.5) (layer Edge.Cuts) (width 0.05))
 (gr_line (start 90 112) (end 101 112) (layer Edge.Cuts) (width 0.05))
 (gr_line (start 90 100) (end 101 100) (layer Edge.Cuts) (width 0.05))
 (gr_line (start 101 96.5) (end 132 96.5) (layer Edge.Cuts) (width 0.05))
 (gr_line (start 90 100) (end 90 112) (layer Edge.Cuts) (width 0.05))
 (segment (start 119.072265 109.703472) (end 119.072249 109.703472) (width 0.2) (layer F.Cu) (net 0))
 (segment (start 94.4 109.5) (end 100.85 109.5) (width 0.6) (layer F.Cu) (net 10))
 (segment (start 102.5 111.15) (end 102.5 114.2) (width 0.6) (layer F.Cu) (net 10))
 (segment (start 100.85 109.5) (end 102.5 111.15) (width 0.6) (layer F.Cu) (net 10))
 (via (at 120.26 104.02) (size 0.45) (drill 0.3) (layers F.Cu B.Cu) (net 2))
 (segment (start 131.03 102.46) (end 131.03 103.39) (width 0.2) (layer F.Cu) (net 2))
 (segment (start 115.9 102.949048) (end 115.9 102.949048) (width 0.2) (layer F.Cu) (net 2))
 (segment (start 94.4 102.5) (end 100.65 102.5) (width 0.6) (layer F.Cu) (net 2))
 (segment (start 100.65 102.5) (end 102.65 100.5) (width 0.6) (layer F.Cu) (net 2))
 (segment (start 102.61 100.46) (end 102.61 97.9) (width 0.6) (layer F.Cu) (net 2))
 (segment (start 102.65 100.5) (end 102.61 100.46) (width 0.6) (layer F.Cu) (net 2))
 (segment (start 102.65 100.5) (end 104.52 100.5) (width 0.4) (layer F.Cu) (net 2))
 (segment (start 104.52 100.5) (end 105.73 100.5) (width 0.4) (layer F.Cu) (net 2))
 (segment (start 105.73 100.5) (end 106.91 100.5) (width 0.4) (layer F.Cu) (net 2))
 (segment (start 107.9 100.5) (end 107.91 100.49) (width 0.4) (layer F.Cu) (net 2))
 (segment (start 106.91 100.5) (end 107.9 100.5) (width 0.4) (layer F.Cu) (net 2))
 (segment (start 107.91 100.49) (end 109.435 100.49) (width 0.4) (layer F.Cu) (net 2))
 (segment (start 109.435 100.49) (end 109.435 100.49) (width 0.4) (layer F.Cu) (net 2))
 (via (at 109.435 100.49) (size 0.45) (drill 0.3) (layers F.Cu B.Cu) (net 2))
 (segment (start 120.822354 101.730843) (end 121.105197 102.013686) (width 0.16) (layer F.Cu) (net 20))
 (segment (start 121.441723 110.32284) (end 121.44284 110.32284) (width 0.2) (layer F.Cu) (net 15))
 (segment (start 121.105197 109.986314) (end 121.441723 110.32284) (width 0.2) (layer F.Cu) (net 15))
 (segment (start 131.03 103.39) (end 131.03 103.39) (width 0.2) (layer F.Cu) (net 2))
 (via (at 131.03 103.39) (size 0.45) (drill 0.3) (layers F.Cu B.Cu) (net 2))
 (segment (start 130.414999 104.005001) (end 128.605001 104.005001) (width 0.2) (layer B.Cu) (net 2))
 (segment (start 131.03 103.39) (end 130.414999 104.005001) (width 0.2) (layer B.Cu) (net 2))
 (segment (start 128.605001 104.005001) (end 126.56 101.96) (width 0.2) (layer B.Cu) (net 2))
 (segment (start 126.56 101.96) (end 120.25 101.96) (width 0.2) (layer B.Cu) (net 2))
 (segment (start 120.25 101.96) (end 120.25 104.02) (width 0.2) (layer B.Cu) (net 2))
 (via (at 115.899993 102.949041) (size 0.45) (drill 0.3) (layers F.Cu B.Cu) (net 2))
 (segment (start 115.900007 102.949041) (end 115.899993 102.949041) (width 0.2) (layer F.Cu) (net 2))
 (segment (start 116.611682 102.237366) (end 115.900007 102.949041) (width 0.2) (layer F.Cu) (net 2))
 (segment (start 109.435 100.49) (end 113.440952 100.49) (width 0.4) (layer B.Cu) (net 2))
 (segment (start 113.440952 100.49) (end 115.899993 102.949041) (width 0.4) (layer B.Cu) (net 2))
 (segment (start 114.878553 103.953553) (end 115.883065 102.949041) (width 0.2) (layer F.Cu) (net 2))
 (segment (start 115.883065 102.949041) (end 115.899993 102.949041) (width 0.2) (layer F.Cu) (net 2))
 (segment (start 119.189041 102.949041) (end 120.26 104.02) (width 0.2) (layer B.Cu) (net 2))
 (segment (start 115.899993 102.949041) (end 119.189041 102.949041) (width 0.2) (layer B.Cu) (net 2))
 (segment (start 131.640001 102.779999) (end 131.03 103.39) (width 0.2) (layer F.Cu) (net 2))
 (segment (start 131.640001 98.160001) (end 131.640001 102.779999) (width 0.2) (layer F.Cu) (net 2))
 (segment (start 131.58 98.1) (end 131.640001 98.160001) (width 0.2) (layer F.Cu) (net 2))
 (segment (start 130.63 98.1) (end 131.58 98.1) (width 0.2) (layer F.Cu) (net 2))
 (segment (start 130.34 98.39) (end 130.63 98.1) (width 0.2) (layer F.Cu) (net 2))
 (segment (start 128.88 98.39) (end 130.34 98.39) (width 0.2) (layer F.Cu) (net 2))
 (segment (start 129.604999 112.135001) (end 129.604999 104.815001) (width 0.2) (layer F.Cu) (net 2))
 (segment (start 126.735 115.005) (end 129.604999 112.135001) (width 0.2) (layer F.Cu) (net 2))
 (segment (start 129.604999 104.815001) (end 131.03 103.39) (width 0.2) (layer F.Cu) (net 2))
 (segment (start 125.735 115.005) (end 126.735 115.005) (width 0.2) (layer F.Cu) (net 2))
 (segment (start 119.355107 102.013686) (end 119.355107 102.005107) (width 0.2) (layer F.Cu) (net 4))
 (segment (start 119.355107 102.005107) (end 119.075 101.725) (width 0.2) (layer F.Cu) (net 4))
 (segment (start 117.525 101.725) (end 117.05 101.25) (width 0.2) (layer F.Cu) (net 4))
 (segment (start 117.05 101.25) (end 116.425 101.25) (width 0.2) (layer F.Cu) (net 4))
 (segment (start 116.425 101.25) (end 115.075 102.6) (width 0.2) (layer F.Cu) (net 4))
 (segment (start 119.071528 102.296528) (end 118.5 101.725) (width 0.2) (layer F.Cu) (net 4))
 (segment (start 119.072265 102.296528) (end 119.071528 102.296528) (width 0.2) (layer F.Cu) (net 4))
 (segment (start 118.5 101.725) (end 117.525 101.725) (width 0.2) (layer F.Cu) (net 4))
 (segment (start 119.075 101.725) (end 118.5 101.725) (width 0.2) (layer F.Cu) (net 4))
 (segment (start 114.817894 102.6) (end 114.171447 103.246447) (width 0.2) (layer F.Cu) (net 4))
 (segment (start 115.075 102.6) (end 114.817894 102.6) (width 0.2) (layer F.Cu) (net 4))
 (segment (start 113.175 102.25) (end 114.171447 103.246447) (width 0.2) (layer F.Cu) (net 4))
 (segment (start 113.175 102.2) (end 113.175 102.25) (width 0.2) (layer F.Cu) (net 4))
 (segment (start 104.52 101.5) (end 105.73 101.5) (width 0.4) (layer F.Cu) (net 3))
 (segment (start 105.73 101.5) (end 106.91 101.5) (width 0.4) (layer F.Cu) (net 3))
 (segment (start 106.91 101.5) (end 111.15 101.5) (width 0.4) (layer F.Cu) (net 3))
 (segment (start 111.15 101.5) (end 111.15 99.95) (width 0.4) (layer F.Cu) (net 3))
 (segment (start 111.425 101.5) (end 112.125 102.2) (width 0.4) (layer F.Cu) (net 3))
 (segment (start 111.15 101.5) (end 111.425 101.5) (width 0.4) (layer F.Cu) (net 3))
 (segment (start 128.88 102.46) (end 130.03 102.46) (width 0.2) (layer F.Cu) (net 11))
 (segment (start 128.88 102.46) (end 128.88 103.52) (width 0.2) (layer F.Cu) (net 11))
 (segment (start 128.88 103.55) (end 128.88 103.55) (width 0.2) (layer F.Cu) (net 11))
 (segment (start 128.88 103.55) (end 128.88 103.55) (width 0.2) (layer F.Cu) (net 11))
 (segment (start 119.63795 101.730843) (end 120.018793 101.35) (width 0.16) (layer F.Cu) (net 11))
 (segment (start 120.018793 101.35) (end 120.018793 101.35) (width 0.16) (layer F.Cu) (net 11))
 (via (at 120.018793 101.35) (size 0.45) (drill 0.3) (layers F.Cu B.Cu) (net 11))
 (segment (start 128.88 103.52) (end 128.88 103.55) (width 0.2) (layer F.Cu) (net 11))
 (via (at 128.88 103.52) (size 0.45) (drill 0.3) (layers F.Cu B.Cu) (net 11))
 (segment (start 126.71 101.35) (end 128.88 103.52) (width 0.16) (layer B.Cu) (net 11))
 (segment (start 120.018793 101.35) (end 126.71 101.35) (width 0.16) (layer B.Cu) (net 11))
 (segment (start 114.925 99.5) (end 114.475 99.95) (width 0.2) (layer F.Cu) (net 7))
 (segment (start 116.525684 99.5) (end 114.925 99.5) (width 0.2) (layer F.Cu) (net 7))
 (segment (start 116.525684 99.5) (end 116.788318 99.762634) (width 0.2) (layer F.Cu) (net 7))
 (segment (start 112.15 99.95) (end 113.475 99.95) (width 0.2) (layer F.Cu) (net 12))
 (segment (start 122.51941 103.427899) (end 122.51941 103.40559) (width 0.2) (layer F.Cu) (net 8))
 (segment (start 122.51941 103.40559) (end 123.225 102.7) (width 0.2) (layer F.Cu) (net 8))
 (segment (start 123.225 102.7) (end 123.225 102.7) (width 0.2) (layer F.Cu) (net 8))
 (via (at 123.225 102.7) (size 0.45) (drill 0.3) (layers F.Cu B.Cu) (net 8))
 (segment (start 95.4 105) (end 99.59 105) (width 0.4) (layer F.Cu) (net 8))
 (segment (start 99.59 105) (end 100.38 104.21) (width 0.4) (layer F.Cu) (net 8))
 (segment (start 100.38 104.21) (end 100.38 104.21) (width 0.4) (layer F.Cu) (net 8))
 (via (at 100.38 104.21) (size 0.45) (drill 0.3) (layers F.Cu B.Cu) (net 8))
 (segment (start 101.98001 105.81001) (end 100.38 104.21) (width 0.2) (layer B.Cu) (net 8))
 (segment (start 120.11499 105.81001) (end 101.98001 105.81001) (width 0.2) (layer B.Cu) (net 8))
 (segment (start 123.225 102.7) (end 120.11499 105.81001) (width 0.2) (layer B.Cu) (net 8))
 (segment (start 122.802253 103.710742) (end 122.814258 103.710742) (width 0.2) (layer F.Cu) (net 9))
 (segment (start 122.858807 103.710742) (end 123.359549 103.21) (width 0.2) (layer F.Cu) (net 9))
 (segment (start 122.802253 103.710742) (end 122.858807 103.710742) (width 0.2) (layer F.Cu) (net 9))
 (segment (start 123.359549 103.21) (end 123.68 103.21) (width 0.2) (layer F.Cu) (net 9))
 (segment (start 123.68 103.21) (end 123.68 103.21) (width 0.2) (layer F.Cu) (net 9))
 (via (at 123.68 103.21) (size 0.45) (drill 0.3) (layers F.Cu B.Cu) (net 9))
 (segment (start 95.4 107) (end 99.61 107) (width 0.4) (layer F.Cu) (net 9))
 (segment (start 99.61 107) (end 99.61 107) (width 0.4) (layer F.Cu) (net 9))
 (via (at 99.61 107) (size 0.45) (drill 0.3) (layers F.Cu B.Cu) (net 9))
 (segment (start 119.89 107) (end 99.61 107) (width 0.2) (layer B.Cu) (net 9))
 (segment (start 123.68 103.21) (end 119.89 107) (width 0.2) (layer B.Cu) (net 9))
 (segment (start 119.402601 99.446447) (end 117.937366 100.911682) (width 0.2) (layer F.Cu) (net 5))
 (segment (start 122.146447 99.446447) (end 119.402601 99.446447) (width 0.2) (layer F.Cu) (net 5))
 (segment (start 121.388039 102.296528) (end 121.724566 101.960001) (width 0.2) (layer F.Cu) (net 6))
 (segment (start 122.853553 100.831014) (end 122.853553 100.153553) (width 0.16) (layer F.Cu) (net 6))
 (segment (start 121.388039 102.296528) (end 122.853553 100.831014) (width 0.16) (layer F.Cu) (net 6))
 (segment (start 130.63 100.3) (end 128.88 100.3) (width 0.2) (layer F.Cu) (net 1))
 (segment (start 128.88 100.3) (end 128.88 101.46) (width 0.2) (layer F.Cu) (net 1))
 (segment (start 128.88 100.3) (end 128.88 99.39) (width 0.2) (layer F.Cu) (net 1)))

